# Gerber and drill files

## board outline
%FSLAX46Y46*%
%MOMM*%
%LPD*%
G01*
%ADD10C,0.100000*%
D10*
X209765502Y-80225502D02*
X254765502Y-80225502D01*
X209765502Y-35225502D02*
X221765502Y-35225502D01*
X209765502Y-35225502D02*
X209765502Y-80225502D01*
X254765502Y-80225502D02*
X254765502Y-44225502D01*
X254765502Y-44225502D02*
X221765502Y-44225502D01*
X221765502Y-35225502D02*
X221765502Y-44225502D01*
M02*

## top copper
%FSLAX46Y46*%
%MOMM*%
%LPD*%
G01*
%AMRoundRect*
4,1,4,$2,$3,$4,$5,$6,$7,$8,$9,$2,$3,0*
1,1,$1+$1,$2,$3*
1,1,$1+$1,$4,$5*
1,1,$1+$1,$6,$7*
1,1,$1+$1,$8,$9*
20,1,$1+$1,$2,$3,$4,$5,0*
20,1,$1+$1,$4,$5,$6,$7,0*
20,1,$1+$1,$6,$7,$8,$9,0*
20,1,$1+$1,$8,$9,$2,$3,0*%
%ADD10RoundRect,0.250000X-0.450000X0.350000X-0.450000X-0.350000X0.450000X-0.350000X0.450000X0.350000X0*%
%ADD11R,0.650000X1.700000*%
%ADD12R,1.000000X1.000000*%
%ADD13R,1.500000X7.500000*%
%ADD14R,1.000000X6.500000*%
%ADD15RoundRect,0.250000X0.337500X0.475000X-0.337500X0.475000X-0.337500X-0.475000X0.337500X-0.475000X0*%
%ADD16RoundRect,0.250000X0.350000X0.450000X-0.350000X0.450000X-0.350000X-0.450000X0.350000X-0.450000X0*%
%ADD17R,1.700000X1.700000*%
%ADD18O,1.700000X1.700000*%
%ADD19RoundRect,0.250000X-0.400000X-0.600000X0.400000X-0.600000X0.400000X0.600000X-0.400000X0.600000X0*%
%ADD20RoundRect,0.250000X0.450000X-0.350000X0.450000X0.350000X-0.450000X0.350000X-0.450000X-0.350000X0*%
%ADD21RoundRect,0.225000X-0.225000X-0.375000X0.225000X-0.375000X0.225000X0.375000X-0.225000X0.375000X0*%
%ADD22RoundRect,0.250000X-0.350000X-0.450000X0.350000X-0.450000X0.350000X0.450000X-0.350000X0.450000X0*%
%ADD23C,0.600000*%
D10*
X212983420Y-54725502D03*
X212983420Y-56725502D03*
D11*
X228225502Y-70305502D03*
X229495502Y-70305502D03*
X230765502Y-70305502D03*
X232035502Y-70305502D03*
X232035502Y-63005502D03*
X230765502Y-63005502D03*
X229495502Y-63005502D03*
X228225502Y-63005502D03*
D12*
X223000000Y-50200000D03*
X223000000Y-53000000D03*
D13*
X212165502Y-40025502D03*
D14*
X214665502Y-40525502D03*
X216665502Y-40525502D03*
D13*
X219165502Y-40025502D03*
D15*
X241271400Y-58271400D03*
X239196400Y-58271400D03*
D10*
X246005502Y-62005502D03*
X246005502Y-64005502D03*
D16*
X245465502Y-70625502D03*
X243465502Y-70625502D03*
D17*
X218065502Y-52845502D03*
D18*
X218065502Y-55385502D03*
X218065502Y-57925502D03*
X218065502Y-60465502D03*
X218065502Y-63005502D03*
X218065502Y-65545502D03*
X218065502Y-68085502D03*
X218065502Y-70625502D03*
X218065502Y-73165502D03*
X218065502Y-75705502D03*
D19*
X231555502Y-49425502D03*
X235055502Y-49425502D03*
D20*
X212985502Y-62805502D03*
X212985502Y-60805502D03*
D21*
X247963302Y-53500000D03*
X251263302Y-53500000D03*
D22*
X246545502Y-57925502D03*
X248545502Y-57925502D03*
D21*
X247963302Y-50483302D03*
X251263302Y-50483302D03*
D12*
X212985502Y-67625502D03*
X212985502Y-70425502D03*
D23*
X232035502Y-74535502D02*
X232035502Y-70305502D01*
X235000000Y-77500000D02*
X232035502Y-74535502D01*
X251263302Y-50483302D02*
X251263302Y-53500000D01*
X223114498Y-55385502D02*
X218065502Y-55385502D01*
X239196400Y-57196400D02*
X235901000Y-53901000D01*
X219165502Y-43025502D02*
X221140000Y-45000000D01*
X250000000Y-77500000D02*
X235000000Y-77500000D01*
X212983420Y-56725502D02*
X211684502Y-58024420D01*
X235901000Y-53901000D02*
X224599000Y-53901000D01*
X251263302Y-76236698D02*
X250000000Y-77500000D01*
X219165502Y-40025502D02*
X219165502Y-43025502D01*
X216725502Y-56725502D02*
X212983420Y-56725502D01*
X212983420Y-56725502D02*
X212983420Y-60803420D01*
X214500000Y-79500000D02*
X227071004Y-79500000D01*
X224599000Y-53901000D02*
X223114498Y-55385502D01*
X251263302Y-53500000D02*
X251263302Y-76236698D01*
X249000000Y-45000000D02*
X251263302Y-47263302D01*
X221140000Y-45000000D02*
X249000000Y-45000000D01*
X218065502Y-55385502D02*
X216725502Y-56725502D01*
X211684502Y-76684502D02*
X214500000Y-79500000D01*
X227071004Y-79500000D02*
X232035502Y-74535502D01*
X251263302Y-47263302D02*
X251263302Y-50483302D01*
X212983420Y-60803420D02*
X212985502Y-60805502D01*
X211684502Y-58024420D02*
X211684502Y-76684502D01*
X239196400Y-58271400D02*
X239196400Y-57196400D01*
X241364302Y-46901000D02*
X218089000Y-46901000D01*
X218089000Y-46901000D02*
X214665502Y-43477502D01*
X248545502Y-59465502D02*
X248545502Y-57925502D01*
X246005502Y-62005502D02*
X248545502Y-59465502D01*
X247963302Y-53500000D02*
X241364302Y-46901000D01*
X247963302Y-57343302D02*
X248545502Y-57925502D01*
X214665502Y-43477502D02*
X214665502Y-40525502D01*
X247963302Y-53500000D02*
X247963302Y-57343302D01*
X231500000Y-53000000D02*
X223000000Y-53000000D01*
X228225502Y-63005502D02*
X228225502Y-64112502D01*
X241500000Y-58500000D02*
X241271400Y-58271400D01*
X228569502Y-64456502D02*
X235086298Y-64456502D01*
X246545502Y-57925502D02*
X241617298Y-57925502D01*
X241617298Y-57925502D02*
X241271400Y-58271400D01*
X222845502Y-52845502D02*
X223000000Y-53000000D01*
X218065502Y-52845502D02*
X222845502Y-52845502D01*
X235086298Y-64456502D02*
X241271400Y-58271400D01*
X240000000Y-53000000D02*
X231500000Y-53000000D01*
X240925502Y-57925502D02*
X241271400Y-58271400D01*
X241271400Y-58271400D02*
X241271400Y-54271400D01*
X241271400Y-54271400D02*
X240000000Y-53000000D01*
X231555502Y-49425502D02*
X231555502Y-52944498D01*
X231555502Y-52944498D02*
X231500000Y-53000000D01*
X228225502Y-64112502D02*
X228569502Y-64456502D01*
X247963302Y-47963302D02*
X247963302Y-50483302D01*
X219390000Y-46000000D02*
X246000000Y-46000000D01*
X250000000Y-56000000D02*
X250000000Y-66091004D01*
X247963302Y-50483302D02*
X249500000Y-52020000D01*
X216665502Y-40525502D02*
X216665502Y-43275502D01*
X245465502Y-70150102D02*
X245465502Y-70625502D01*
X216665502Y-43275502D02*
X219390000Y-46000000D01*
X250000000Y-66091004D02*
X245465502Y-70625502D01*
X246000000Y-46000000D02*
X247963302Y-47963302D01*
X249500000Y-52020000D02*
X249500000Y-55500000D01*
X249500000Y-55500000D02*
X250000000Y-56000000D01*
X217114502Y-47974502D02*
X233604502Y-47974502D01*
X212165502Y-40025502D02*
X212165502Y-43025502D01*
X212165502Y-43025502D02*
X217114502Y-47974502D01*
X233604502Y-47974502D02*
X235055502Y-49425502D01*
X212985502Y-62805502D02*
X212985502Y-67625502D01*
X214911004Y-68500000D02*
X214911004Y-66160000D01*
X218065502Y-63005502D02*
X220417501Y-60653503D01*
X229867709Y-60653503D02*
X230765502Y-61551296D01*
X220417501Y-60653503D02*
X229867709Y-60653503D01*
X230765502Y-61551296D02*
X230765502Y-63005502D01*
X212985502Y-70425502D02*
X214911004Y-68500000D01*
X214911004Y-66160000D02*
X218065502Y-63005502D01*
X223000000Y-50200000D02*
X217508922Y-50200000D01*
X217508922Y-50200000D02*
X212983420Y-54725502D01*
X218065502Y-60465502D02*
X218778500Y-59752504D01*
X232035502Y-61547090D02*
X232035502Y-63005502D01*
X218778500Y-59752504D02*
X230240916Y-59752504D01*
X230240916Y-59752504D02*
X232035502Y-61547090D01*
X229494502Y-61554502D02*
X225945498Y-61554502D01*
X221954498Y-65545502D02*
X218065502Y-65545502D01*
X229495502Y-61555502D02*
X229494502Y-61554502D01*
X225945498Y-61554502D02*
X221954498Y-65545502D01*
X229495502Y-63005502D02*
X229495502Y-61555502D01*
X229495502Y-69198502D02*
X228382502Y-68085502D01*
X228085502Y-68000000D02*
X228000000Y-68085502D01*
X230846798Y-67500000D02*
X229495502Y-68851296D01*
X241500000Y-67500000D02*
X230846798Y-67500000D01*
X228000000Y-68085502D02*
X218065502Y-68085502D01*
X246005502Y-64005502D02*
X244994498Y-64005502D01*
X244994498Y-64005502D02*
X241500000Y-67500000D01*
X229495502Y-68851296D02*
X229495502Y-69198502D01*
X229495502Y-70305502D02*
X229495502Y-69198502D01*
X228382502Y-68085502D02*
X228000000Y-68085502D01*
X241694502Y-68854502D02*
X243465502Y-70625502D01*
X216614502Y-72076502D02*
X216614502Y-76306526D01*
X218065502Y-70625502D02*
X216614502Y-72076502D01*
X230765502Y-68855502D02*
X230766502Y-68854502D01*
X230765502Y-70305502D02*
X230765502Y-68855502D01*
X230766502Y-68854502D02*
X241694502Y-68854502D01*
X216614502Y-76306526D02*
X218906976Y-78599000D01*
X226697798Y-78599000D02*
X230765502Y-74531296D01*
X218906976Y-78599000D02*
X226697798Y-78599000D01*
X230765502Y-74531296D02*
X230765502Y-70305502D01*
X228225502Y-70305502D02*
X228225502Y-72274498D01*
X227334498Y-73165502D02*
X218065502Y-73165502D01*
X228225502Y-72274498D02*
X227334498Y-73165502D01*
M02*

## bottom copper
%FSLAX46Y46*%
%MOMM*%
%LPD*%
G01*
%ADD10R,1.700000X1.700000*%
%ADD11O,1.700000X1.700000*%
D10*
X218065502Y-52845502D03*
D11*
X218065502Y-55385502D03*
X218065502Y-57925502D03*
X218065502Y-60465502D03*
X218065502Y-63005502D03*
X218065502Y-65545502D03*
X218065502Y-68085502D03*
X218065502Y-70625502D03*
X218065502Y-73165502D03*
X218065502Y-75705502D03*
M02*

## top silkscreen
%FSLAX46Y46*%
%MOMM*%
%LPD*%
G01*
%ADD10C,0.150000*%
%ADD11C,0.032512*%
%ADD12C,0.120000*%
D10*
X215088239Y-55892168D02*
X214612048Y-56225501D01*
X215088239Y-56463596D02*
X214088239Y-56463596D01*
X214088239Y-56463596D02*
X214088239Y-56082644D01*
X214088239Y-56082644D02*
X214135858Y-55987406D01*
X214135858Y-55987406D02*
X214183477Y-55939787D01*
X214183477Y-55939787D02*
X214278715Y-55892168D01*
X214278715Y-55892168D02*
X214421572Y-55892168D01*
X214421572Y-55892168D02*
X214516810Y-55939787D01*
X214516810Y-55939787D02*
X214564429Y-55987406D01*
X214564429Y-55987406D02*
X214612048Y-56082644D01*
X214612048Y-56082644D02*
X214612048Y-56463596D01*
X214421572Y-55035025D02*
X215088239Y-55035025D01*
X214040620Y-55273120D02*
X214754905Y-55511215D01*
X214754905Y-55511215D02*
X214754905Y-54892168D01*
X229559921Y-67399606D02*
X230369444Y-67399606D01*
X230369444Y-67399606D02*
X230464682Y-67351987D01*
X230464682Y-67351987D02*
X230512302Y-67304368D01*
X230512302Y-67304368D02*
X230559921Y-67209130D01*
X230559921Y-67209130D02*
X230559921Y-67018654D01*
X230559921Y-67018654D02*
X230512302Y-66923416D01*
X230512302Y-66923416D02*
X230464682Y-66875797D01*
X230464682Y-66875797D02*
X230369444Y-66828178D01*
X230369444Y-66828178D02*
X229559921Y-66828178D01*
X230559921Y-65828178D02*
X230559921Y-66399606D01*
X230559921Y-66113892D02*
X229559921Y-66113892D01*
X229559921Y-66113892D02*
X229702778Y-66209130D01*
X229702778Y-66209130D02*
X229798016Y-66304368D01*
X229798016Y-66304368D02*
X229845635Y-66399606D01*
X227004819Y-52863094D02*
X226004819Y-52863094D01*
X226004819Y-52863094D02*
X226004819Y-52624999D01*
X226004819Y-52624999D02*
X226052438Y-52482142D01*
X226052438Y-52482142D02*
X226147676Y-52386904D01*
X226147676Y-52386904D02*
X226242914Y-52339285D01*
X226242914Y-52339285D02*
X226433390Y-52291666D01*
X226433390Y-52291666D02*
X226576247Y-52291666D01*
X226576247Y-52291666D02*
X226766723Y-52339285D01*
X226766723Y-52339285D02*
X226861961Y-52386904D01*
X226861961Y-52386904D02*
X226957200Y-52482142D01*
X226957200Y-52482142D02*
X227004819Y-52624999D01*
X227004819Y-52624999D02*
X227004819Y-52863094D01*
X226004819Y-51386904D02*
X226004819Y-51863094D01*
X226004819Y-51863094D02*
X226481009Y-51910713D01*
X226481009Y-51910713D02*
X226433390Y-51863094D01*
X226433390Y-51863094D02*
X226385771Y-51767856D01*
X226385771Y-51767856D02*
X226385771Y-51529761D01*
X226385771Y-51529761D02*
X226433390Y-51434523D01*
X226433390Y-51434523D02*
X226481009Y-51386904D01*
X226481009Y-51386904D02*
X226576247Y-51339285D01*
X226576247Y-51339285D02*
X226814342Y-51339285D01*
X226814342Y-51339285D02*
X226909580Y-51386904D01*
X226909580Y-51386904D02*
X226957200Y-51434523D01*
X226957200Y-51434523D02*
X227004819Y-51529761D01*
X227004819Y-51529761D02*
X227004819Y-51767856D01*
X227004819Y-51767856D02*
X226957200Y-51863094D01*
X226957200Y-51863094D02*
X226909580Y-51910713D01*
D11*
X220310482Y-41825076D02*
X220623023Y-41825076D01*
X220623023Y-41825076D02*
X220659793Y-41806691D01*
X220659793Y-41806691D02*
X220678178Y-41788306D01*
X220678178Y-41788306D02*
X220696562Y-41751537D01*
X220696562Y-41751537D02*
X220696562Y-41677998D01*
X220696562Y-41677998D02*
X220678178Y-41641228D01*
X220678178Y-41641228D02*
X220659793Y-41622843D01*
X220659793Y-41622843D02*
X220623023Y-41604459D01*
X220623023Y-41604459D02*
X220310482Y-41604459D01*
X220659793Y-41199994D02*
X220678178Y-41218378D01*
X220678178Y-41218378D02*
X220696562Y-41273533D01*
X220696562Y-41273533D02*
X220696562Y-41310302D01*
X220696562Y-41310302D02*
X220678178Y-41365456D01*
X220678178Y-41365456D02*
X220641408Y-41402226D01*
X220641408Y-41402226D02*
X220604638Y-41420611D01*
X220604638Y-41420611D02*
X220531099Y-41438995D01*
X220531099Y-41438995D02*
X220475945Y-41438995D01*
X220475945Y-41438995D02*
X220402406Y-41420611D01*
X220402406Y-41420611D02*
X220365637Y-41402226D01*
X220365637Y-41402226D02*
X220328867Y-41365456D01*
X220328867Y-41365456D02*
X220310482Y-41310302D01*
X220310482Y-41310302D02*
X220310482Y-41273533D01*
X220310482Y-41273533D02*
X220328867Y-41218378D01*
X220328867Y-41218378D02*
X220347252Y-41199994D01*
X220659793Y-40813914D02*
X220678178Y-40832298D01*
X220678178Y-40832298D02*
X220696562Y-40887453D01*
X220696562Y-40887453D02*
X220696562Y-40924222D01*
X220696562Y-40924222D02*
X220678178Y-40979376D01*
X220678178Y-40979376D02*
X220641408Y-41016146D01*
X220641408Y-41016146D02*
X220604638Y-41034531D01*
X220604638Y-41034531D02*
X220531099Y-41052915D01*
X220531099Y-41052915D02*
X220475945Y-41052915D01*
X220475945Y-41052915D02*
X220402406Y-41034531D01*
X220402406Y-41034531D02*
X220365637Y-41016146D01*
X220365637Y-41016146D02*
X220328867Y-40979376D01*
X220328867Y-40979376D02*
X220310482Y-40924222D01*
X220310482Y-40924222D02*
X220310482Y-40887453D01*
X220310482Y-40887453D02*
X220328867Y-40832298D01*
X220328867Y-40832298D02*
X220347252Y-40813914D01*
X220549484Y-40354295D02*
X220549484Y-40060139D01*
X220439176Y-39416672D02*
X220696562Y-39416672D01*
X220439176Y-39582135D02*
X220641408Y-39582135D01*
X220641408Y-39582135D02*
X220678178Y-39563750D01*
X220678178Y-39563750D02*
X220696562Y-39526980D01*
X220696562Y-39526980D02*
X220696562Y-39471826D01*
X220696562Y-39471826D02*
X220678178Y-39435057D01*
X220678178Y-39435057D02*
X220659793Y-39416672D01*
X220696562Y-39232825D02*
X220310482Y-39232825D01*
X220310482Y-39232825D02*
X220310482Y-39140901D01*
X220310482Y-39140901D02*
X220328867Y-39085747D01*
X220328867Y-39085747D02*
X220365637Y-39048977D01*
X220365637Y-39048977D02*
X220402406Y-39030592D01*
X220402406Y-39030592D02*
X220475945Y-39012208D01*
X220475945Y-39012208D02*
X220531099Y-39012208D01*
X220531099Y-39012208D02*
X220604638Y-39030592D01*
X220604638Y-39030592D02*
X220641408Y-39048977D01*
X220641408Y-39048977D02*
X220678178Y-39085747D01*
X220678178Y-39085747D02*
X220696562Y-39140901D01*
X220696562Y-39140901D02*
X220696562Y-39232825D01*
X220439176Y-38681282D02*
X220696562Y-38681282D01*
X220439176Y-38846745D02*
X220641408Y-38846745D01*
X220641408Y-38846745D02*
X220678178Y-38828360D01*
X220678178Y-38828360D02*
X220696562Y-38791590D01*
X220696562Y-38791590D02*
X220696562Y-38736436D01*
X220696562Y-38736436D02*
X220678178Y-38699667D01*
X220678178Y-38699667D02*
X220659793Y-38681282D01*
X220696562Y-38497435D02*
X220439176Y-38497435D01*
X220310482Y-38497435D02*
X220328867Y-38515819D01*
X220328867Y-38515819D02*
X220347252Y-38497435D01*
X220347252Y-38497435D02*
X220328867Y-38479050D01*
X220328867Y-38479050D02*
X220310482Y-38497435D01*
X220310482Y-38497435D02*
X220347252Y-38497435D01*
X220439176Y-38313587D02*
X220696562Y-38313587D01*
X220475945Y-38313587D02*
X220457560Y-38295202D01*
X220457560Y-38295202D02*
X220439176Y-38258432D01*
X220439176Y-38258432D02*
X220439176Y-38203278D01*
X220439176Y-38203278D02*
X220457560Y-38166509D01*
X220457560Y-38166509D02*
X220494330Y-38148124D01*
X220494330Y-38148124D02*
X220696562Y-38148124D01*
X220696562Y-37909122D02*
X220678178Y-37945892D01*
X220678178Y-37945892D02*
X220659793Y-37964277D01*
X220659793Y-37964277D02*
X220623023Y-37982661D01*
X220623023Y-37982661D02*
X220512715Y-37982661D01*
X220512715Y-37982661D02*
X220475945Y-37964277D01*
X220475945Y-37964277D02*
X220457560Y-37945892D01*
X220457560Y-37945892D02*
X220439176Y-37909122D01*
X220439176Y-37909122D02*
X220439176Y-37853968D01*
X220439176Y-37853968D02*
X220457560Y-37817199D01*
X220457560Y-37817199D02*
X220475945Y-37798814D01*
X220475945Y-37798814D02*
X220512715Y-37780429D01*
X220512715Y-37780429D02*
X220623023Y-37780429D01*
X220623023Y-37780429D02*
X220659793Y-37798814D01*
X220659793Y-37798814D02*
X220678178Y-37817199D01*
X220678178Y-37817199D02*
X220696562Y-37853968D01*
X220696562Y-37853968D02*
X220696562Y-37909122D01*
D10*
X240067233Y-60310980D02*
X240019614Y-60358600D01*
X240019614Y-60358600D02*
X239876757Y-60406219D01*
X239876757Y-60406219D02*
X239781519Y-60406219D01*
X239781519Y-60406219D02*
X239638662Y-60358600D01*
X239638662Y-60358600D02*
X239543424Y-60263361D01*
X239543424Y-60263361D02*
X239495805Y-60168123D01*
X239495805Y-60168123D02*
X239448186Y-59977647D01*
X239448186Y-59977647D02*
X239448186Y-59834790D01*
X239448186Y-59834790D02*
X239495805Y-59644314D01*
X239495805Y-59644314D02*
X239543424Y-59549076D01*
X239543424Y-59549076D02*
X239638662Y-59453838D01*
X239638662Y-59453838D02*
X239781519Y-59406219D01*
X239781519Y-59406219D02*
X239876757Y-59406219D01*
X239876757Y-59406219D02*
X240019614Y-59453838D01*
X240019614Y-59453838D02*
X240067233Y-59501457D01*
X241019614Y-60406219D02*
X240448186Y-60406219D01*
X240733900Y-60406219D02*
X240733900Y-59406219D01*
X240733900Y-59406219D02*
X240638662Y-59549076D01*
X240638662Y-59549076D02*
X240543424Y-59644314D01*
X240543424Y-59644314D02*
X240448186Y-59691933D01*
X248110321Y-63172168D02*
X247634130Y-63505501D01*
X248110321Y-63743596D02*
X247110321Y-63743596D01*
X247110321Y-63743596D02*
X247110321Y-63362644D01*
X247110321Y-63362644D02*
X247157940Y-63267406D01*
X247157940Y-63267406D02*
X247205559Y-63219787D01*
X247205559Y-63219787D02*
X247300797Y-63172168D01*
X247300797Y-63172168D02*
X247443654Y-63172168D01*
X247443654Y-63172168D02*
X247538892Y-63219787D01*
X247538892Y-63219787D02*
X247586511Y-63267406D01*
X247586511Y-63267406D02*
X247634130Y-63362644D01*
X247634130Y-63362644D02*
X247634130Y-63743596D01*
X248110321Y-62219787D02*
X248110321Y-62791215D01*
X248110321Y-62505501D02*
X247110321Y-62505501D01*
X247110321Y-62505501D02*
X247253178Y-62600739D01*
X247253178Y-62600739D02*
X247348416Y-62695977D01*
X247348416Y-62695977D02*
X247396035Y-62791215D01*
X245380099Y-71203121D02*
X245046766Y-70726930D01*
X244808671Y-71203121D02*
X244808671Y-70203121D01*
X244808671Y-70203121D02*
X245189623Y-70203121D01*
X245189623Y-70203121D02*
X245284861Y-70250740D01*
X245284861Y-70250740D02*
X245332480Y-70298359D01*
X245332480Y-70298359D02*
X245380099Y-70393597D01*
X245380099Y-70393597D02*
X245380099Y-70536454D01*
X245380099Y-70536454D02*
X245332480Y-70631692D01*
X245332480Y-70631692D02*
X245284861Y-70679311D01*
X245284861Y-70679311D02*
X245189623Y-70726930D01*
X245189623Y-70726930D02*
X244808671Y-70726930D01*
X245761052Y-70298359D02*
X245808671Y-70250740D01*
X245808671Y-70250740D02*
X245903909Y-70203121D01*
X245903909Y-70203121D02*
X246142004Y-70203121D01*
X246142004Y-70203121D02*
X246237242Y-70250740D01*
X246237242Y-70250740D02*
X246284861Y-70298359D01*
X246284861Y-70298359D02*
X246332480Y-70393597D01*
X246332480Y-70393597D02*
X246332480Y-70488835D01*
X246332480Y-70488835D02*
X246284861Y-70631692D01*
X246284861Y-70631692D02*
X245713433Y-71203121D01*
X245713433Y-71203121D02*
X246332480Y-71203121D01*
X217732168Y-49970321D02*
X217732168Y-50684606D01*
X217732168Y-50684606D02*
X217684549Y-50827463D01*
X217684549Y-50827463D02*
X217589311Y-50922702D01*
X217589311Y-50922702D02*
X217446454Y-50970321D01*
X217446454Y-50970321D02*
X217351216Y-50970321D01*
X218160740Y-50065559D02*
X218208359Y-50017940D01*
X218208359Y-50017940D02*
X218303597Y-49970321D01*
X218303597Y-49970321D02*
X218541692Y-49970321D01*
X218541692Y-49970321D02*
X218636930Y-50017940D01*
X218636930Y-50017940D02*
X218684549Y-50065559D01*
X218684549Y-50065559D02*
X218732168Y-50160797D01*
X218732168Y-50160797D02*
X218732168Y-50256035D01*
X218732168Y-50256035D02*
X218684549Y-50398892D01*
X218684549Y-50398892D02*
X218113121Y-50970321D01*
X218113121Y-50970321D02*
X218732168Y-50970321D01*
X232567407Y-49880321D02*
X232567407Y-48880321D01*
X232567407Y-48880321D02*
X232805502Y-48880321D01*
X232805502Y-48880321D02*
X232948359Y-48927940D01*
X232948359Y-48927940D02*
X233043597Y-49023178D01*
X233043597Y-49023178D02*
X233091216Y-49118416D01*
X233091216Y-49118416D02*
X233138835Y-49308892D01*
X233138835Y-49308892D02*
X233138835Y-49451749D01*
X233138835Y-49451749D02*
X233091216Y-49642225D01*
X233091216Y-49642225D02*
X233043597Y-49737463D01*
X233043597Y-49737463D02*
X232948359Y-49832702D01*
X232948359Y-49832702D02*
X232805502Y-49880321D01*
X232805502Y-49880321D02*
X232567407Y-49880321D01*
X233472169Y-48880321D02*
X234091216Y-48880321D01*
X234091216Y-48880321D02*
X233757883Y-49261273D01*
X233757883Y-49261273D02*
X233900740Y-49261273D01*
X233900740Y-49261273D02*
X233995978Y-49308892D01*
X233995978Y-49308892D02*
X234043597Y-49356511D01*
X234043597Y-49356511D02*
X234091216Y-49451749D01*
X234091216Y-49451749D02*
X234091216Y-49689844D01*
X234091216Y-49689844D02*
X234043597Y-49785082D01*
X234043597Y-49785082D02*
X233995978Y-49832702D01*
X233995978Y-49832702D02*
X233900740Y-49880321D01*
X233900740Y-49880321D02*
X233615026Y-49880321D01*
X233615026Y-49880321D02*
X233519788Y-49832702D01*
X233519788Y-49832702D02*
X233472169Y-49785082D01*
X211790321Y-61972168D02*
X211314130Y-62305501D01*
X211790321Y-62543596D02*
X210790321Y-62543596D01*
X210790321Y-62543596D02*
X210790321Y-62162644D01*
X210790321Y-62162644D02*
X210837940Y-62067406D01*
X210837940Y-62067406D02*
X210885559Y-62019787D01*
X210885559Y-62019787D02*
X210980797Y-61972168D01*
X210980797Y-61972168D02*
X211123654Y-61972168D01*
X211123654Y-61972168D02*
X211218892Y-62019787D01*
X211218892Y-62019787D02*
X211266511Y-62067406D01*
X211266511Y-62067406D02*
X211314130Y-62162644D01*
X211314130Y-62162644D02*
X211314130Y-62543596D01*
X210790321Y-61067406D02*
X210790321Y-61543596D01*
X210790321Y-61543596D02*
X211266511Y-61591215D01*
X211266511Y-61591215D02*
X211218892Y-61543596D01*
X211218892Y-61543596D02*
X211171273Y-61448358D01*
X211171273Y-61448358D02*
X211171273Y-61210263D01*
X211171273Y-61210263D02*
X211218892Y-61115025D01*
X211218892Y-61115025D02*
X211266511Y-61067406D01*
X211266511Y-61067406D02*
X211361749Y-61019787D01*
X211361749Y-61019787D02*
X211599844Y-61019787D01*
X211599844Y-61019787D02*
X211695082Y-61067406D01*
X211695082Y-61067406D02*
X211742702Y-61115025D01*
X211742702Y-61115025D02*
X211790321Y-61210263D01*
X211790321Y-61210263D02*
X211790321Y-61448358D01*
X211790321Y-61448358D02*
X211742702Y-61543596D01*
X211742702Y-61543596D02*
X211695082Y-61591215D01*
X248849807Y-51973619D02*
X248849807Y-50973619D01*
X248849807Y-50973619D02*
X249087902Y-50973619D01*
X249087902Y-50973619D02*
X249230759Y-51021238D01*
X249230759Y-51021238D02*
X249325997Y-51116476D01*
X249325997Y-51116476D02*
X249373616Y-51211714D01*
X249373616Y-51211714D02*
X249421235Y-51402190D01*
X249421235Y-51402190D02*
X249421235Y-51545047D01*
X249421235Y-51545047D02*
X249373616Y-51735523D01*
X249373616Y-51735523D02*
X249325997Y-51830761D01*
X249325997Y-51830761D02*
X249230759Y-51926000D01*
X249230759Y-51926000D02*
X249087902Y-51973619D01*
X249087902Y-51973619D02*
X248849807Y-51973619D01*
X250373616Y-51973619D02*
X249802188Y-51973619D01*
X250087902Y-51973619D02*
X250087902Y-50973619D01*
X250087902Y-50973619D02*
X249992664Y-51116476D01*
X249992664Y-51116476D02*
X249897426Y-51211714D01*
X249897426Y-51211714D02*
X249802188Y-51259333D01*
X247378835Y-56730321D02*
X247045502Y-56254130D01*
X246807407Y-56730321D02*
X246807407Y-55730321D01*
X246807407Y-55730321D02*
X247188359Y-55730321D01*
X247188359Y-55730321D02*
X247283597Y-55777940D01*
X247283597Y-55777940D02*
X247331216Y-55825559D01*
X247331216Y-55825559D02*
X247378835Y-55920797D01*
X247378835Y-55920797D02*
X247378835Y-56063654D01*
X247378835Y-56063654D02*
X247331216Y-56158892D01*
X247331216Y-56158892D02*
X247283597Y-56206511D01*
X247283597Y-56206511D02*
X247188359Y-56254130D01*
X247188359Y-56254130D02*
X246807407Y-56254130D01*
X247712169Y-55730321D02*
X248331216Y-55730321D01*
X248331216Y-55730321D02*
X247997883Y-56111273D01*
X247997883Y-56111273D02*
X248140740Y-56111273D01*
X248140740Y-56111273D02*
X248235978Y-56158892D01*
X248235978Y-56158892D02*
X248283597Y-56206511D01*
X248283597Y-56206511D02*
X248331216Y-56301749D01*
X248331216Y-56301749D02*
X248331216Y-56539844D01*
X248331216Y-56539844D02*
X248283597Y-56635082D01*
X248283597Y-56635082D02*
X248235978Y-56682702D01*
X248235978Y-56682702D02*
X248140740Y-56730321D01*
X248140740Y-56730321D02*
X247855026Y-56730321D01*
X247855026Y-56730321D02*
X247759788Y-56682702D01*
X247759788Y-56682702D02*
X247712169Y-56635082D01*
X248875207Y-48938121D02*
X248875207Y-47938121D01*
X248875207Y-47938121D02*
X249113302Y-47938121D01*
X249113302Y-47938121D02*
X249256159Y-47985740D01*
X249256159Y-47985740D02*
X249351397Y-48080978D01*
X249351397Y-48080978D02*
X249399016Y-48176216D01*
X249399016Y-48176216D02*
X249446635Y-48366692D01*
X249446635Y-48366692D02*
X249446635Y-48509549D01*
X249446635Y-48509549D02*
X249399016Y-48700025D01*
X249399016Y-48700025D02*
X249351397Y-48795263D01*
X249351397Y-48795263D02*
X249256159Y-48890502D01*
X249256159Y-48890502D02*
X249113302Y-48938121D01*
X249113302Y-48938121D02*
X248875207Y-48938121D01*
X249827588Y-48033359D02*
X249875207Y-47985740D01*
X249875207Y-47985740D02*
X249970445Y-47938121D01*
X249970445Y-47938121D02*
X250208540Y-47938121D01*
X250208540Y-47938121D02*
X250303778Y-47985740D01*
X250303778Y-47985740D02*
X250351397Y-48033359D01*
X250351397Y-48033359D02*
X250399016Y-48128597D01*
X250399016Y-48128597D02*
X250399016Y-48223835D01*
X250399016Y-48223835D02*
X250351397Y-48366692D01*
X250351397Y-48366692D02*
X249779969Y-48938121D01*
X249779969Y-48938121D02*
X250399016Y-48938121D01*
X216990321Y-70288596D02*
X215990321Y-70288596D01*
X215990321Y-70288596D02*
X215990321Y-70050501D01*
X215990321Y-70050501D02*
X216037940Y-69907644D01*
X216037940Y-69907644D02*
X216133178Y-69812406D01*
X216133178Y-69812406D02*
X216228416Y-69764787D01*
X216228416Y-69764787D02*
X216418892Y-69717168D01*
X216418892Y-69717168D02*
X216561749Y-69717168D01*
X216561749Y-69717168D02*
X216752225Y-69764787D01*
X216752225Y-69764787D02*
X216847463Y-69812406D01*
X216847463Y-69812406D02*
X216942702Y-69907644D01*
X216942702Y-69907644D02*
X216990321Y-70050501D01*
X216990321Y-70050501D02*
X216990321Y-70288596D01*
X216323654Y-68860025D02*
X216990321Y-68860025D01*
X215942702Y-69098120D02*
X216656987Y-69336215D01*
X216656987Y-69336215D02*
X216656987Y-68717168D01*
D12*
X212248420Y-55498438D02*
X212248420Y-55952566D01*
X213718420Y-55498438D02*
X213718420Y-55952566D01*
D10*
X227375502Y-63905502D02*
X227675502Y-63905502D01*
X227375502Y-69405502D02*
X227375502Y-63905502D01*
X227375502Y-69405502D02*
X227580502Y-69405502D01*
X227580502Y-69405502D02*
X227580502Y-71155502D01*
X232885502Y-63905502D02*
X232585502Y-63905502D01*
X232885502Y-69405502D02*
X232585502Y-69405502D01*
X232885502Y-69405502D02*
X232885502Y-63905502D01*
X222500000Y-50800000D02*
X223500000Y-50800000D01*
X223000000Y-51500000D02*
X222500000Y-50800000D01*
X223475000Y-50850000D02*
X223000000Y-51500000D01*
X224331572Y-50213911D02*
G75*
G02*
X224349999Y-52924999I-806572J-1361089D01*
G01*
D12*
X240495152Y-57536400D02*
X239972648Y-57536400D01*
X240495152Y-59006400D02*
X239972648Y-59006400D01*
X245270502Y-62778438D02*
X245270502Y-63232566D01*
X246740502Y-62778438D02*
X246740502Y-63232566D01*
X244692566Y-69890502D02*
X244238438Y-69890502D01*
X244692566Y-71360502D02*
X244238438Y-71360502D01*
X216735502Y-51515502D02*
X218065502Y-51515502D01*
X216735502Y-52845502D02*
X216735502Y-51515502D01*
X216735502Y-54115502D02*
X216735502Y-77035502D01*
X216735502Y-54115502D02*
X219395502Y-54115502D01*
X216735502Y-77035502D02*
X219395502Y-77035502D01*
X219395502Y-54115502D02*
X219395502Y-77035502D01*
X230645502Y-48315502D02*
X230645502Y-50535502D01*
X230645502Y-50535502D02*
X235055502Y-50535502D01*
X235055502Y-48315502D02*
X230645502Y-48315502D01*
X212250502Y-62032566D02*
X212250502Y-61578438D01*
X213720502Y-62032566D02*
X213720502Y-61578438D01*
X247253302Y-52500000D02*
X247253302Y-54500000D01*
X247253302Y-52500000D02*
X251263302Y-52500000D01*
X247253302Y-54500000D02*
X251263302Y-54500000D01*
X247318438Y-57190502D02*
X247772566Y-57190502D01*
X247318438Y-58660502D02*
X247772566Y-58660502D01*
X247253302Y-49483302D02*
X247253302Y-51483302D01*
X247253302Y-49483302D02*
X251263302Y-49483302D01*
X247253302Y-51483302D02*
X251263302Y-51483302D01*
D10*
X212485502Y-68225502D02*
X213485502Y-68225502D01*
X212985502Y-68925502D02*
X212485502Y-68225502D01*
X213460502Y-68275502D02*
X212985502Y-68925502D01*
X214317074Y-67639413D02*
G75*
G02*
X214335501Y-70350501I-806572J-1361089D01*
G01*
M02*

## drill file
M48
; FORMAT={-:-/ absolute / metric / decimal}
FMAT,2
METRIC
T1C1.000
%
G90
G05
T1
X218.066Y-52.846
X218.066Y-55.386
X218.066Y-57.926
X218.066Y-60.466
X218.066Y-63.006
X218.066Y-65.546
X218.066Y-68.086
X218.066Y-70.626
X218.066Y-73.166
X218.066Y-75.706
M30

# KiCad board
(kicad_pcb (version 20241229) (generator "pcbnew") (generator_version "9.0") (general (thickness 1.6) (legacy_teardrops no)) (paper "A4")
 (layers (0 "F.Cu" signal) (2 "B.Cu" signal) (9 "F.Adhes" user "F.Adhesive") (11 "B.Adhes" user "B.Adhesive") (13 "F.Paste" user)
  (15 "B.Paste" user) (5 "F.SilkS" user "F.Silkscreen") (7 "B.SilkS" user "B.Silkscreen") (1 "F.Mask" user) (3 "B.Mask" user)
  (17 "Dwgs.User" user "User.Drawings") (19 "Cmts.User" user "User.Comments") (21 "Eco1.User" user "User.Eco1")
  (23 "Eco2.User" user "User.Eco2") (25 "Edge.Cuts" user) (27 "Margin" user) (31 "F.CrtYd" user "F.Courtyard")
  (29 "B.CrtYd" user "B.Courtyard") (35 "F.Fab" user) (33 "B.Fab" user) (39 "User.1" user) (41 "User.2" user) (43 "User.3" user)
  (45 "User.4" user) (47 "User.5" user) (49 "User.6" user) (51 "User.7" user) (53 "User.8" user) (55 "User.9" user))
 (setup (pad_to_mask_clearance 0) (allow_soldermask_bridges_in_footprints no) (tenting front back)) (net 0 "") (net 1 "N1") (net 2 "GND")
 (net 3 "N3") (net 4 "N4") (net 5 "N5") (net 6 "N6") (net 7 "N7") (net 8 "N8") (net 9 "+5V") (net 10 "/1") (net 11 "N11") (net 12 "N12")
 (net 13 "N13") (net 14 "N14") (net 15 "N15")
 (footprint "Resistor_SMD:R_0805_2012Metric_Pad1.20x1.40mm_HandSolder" (layer "F.Cu") (at 212.98342 55.725502 -90)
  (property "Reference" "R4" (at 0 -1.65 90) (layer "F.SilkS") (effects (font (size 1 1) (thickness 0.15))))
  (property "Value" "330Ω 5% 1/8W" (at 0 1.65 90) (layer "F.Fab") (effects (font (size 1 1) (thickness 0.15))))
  (fp_line (start -0.227064 0.735) (end 0.227064 0.735) (stroke (width 0.12) (type solid)) (layer "F.SilkS"))
  (fp_line (start -0.227064 -0.735) (end 0.227064 -0.735) (stroke (width 0.12) (type solid)) (layer "F.SilkS"))
  (pad "1" smd roundrect (at -1 0 270) (size 1.2 1.4) (layers "F.Cu" "F.Mask" "F.Paste") (roundrect_rratio 0.208333) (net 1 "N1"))
  (pad "2" smd roundrect (at 1 0 270) (size 1.2 1.4) (layers "F.Cu" "F.Mask" "F.Paste") (roundrect_rratio 0.208333) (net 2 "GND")))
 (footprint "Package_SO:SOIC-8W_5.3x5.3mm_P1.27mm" (layer "F.Cu") (at 230.130502 66.655502 90)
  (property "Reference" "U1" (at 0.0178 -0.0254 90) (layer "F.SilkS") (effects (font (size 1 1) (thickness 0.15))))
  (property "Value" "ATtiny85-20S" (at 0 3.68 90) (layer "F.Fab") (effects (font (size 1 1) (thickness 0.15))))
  (fp_line (start 2.75 -2.755) (end 2.75 -2.455) (stroke (width 0.15) (type solid)) (layer "F.SilkS"))
  (fp_line (start -2.75 -2.755) (end 2.75 -2.755) (stroke (width 0.15) (type solid)) (layer "F.SilkS"))
  (fp_line (start -2.75 -2.755) (end -2.75 -2.55) (stroke (width 0.15) (type solid)) (layer "F.SilkS"))
  (fp_line (start -2.75 -2.55) (end -4.5 -2.55) (stroke (width 0.15) (type solid)) (layer "F.SilkS"))
  (fp_line (start 2.75 2.755) (end 2.75 2.455) (stroke (width 0.15) (type solid)) (layer "F.SilkS"))
  (fp_line (start -2.75 2.755) (end -2.75 2.455) (stroke (width 0.15) (type solid)) (layer "F.SilkS"))
  (fp_line (start -2.75 2.755) (end 2.75 2.755) (stroke (width 0.15) (type solid)) (layer "F.SilkS"))
  (pad "1" smd rect (at -3.65 -1.905 90) (size 1.7 0.65) (layers "F.Cu" "F.Mask" "F.Paste") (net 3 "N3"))
  (pad "2" smd rect (at -3.65 -0.635 90) (size 1.7 0.65) (layers "F.Cu" "F.Mask" "F.Paste") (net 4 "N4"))
  (pad "3" smd rect (at -3.65 0.635 90) (size 1.7 0.65) (layers "F.Cu" "F.Mask" "F.Paste") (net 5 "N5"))
  (pad "4" smd rect (at -3.65 1.905 90) (size 1.7 0.65) (layers "F.Cu" "F.Mask" "F.Paste") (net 2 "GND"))
  (pad "5" smd rect (at 3.65 1.905 90) (size 1.7 0.65) (layers "F.Cu" "F.Mask" "F.Paste") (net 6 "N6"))
  (pad "6" smd rect (at 3.65 0.635 90) (size 1.7 0.65) (layers "F.Cu" "F.Mask" "F.Paste") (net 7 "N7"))
  (pad "7" smd rect (at 3.65 -0.635 90) (size 1.7 0.65) (layers "F.Cu" "F.Mask" "F.Paste") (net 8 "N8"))
  (pad "8" smd rect (at 3.65 -1.905 90) (size 1.7 0.65) (layers "F.Cu" "F.Mask" "F.Paste") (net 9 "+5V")))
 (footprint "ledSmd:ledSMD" (layer "F.Cu") (at 223 52 -90)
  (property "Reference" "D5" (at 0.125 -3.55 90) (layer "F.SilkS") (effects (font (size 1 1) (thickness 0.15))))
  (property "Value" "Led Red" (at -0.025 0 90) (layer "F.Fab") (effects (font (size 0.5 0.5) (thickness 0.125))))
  (fp_line (start -1.2 0.5) (end -1.2 -0.5) (stroke (width 0.15) (type solid)) (layer "F.SilkS"))
  (fp_line (start -0.5 0) (end -1.2 0.5) (stroke (width 0.15) (type solid)) (layer "F.SilkS"))
  (fp_line (start -1.15 -0.475) (end -0.5 0) (stroke (width 0.15) (type solid)) (layer "F.SilkS"))
  (fp_arc (start -1.786089 -1.331572) (mid -0.435753 -2.107089) (end 0.924999 -1.349999) (stroke (width 0.15) (type solid))
   (layer "F.SilkS"))
  (pad "1" smd rect (at -1.8 0 270) (size 1 1) (layers "F.Cu" "F.Mask" "F.Paste") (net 1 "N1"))
  (pad "2" smd rect (at 1 0 270) (size 1 1) (layers "F.Cu" "F.Mask" "F.Paste") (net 9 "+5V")))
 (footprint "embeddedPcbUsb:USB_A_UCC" (layer "F.Cu") (at 215.665502 40.225502 -90)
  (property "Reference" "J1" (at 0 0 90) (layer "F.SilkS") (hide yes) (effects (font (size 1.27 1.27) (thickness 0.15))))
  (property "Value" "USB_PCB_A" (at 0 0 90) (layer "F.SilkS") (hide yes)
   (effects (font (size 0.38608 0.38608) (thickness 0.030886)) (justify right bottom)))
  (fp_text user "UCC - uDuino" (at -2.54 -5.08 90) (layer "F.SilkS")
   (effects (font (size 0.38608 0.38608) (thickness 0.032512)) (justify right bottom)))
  (pad "1" smd rect (at -0.2 3.5 270) (size 7.5 1.5) (layers "F.Cu" "F.Mask" "F.Paste") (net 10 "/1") (solder_mask_margin 0.1016))
  (pad "2" smd rect (at 0.3 1 270) (size 6.5 1) (layers "F.Cu" "F.Mask" "F.Paste") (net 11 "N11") (solder_mask_margin 0.1016))
  (pad "3" smd rect (at 0.3 -1 270) (size 6.5 1) (layers "F.Cu" "F.Mask" "F.Paste") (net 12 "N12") (solder_mask_margin 0.1016))
  (pad "4" smd rect (at -0.2 -3.5 270) (size 7.5 1.5) (layers "F.Cu" "F.Mask" "F.Paste") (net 2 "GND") (solder_mask_margin 0.1016)))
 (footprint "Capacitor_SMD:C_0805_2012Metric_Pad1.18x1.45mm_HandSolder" (layer "F.Cu") (at 240.2339 58.2714 180)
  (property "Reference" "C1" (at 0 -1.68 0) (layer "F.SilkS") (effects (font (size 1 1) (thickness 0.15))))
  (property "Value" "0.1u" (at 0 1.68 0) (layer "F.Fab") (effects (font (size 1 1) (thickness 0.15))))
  (fp_line (start -0.261252 0.735) (end 0.261252 0.735) (stroke (width 0.12) (type solid)) (layer "F.SilkS"))
  (fp_line (start -0.261252 -0.735) (end 0.261252 -0.735) (stroke (width 0.12) (type solid)) (layer "F.SilkS"))
  (pad "1" smd roundrect (at -1.0375 0 180) (size 1.175 1.45) (layers "F.Cu" "F.Mask" "F.Paste") (roundrect_rratio 0.212766) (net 9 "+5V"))
  (pad "2" smd roundrect (at 1.0375 0 180) (size 1.175 1.45) (layers "F.Cu" "F.Mask" "F.Paste") (roundrect_rratio 0.212766) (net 2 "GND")))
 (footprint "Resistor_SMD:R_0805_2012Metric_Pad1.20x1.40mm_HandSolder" (layer "F.Cu") (at 246.005502 63.005502 -90)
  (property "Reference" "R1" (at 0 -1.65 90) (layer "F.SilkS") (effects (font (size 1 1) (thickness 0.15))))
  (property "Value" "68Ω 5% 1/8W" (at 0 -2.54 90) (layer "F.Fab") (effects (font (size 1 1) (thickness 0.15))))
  (fp_line (start -0.227064 0.735) (end 0.227064 0.735) (stroke (width 0.12) (type solid)) (layer "F.SilkS"))
  (fp_line (start -0.227064 -0.735) (end 0.227064 -0.735) (stroke (width 0.12) (type solid)) (layer "F.SilkS"))
  (pad "1" smd roundrect (at -1 0 270) (size 1.2 1.4) (layers "F.Cu" "F.Mask" "F.Paste") (roundrect_rratio 0.208333) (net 11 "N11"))
  (pad "2" smd roundrect (at 1 0 270) (size 1.2 1.4) (layers "F.Cu" "F.Mask" "F.Paste") (roundrect_rratio 0.208333) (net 4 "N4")))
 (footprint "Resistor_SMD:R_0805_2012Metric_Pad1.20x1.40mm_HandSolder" (layer "F.Cu") (at 244.465502 70.625502 180)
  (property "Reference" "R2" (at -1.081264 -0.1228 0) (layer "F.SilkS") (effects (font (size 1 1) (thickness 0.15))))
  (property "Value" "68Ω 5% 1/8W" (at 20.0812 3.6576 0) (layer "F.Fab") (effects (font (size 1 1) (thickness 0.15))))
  (fp_line (start -0.227064 0.735) (end 0.227064 0.735) (stroke (width 0.12) (type solid)) (layer "F.SilkS"))
  (fp_line (start -0.227064 -0.735) (end 0.227064 -0.735) (stroke (width 0.12) (type solid)) (layer "F.SilkS"))
  (pad "1" smd roundrect (at -1 0 180) (size 1.2 1.4) (layers "F.Cu" "F.Mask" "F.Paste") (roundrect_rratio 0.208333) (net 12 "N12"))
  (pad "2" smd roundrect (at 1 0 180) (size 1.2 1.4) (layers "F.Cu" "F.Mask" "F.Paste") (roundrect_rratio 0.208333) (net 5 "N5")))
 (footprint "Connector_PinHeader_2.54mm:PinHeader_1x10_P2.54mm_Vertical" (layer "F.Cu") (at 218.065502 52.845502)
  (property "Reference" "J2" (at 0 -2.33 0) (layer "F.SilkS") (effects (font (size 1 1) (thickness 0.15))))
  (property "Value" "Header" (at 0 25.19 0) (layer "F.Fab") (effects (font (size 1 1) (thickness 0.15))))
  (fp_line (start -1.33 -1.33) (end 0 -1.33) (stroke (width 0.12) (type solid)) (layer "F.SilkS"))
  (fp_line (start -1.33 0) (end -1.33 -1.33) (stroke (width 0.12) (type solid)) (layer "F.SilkS"))
  (fp_line (start -1.33 1.27) (end -1.33 24.19) (stroke (width 0.12) (type solid)) (layer "F.SilkS"))
  (fp_line (start -1.33 1.27) (end 1.33 1.27) (stroke (width 0.12) (type solid)) (layer "F.SilkS"))
  (fp_line (start -1.33 24.19) (end 1.33 24.19) (stroke (width 0.12) (type solid)) (layer "F.SilkS"))
  (fp_line (start 1.33 1.27) (end 1.33 24.19) (stroke (width 0.12) (type solid)) (layer "F.SilkS"))
  (pad "1" thru_hole rect (at 0 0) (size 1.7 1.7) (drill 1) (layers "*.Cu" "*.Mask") (remove_unused_layers no) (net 9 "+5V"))
  (pad "2" thru_hole oval (at 0 2.54) (size 1.7 1.7) (drill 1) (layers "*.Cu" "*.Mask") (remove_unused_layers no) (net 2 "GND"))
  (pad "3" thru_hole oval (at 0 5.08) (size 1.7 1.7) (drill 1) (layers "*.Cu" "*.Mask") (remove_unused_layers no) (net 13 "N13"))
  (pad "4" thru_hole oval (at 0 7.62) (size 1.7 1.7) (drill 1) (layers "*.Cu" "*.Mask") (remove_unused_layers no) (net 6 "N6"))
  (pad "5" thru_hole oval (at 0 10.16) (size 1.7 1.7) (drill 1) (layers "*.Cu" "*.Mask") (remove_unused_layers no) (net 7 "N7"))
  (pad "6" thru_hole oval (at 0 12.7) (size 1.7 1.7) (drill 1) (layers "*.Cu" "*.Mask") (remove_unused_layers no) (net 8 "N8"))
  (pad "7" thru_hole oval (at 0 15.24) (size 1.7 1.7) (drill 1) (layers "*.Cu" "*.Mask") (remove_unused_layers no) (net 4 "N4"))
  (pad "8" thru_hole oval (at 0 17.78) (size 1.7 1.7) (drill 1) (layers "*.Cu" "*.Mask") (remove_unused_layers no) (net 5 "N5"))
  (pad "9" thru_hole oval (at 0 20.32) (size 1.7 1.7) (drill 1) (layers "*.Cu" "*.Mask") (remove_unused_layers no) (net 3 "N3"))
  (pad "10" thru_hole oval (at 0 22.86) (size 1.7 1.7) (drill 1) (layers "*.Cu" "*.Mask") (remove_unused_layers no) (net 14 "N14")))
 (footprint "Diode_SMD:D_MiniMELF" (layer "F.Cu") (at 233.305502 49.425502)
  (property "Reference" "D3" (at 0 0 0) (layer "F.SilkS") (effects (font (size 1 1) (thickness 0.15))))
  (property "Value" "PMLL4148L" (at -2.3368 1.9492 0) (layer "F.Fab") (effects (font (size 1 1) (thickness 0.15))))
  (fp_line (start -2.66 -1.11) (end -2.66 1.11) (stroke (width 0.12) (type solid)) (layer "F.SilkS"))
  (fp_line (start -2.66 1.11) (end 1.75 1.11) (stroke (width 0.12) (type solid)) (layer "F.SilkS"))
  (fp_line (start 1.75 -1.11) (end -2.66 -1.11) (stroke (width 0.12) (type solid)) (layer "F.SilkS"))
  (pad "1" smd roundrect (at -1.75 0) (size 1.3 1.7) (layers "F.Cu" "F.Mask" "F.Paste") (roundrect_rratio 0.1923076923) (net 9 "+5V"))
  (pad "2" smd roundrect (at 1.75 0) (size 1.3 1.7) (layers "F.Cu" "F.Mask" "F.Paste") (roundrect_rratio 0.1923076923) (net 10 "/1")))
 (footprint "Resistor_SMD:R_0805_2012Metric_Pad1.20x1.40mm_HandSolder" (layer "F.Cu") (at 212.985502 61.805502 90)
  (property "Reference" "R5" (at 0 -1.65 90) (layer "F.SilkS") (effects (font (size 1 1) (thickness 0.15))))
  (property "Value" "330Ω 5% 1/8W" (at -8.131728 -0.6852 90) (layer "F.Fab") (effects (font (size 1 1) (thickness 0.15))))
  (fp_line (start -0.227064 -0.735) (end 0.227064 -0.735) (stroke (width 0.12) (type solid)) (layer "F.SilkS"))
  (fp_line (start -0.227064 0.735) (end 0.227064 0.735) (stroke (width 0.12) (type solid)) (layer "F.SilkS"))
  (pad "1" smd roundrect (at -1 0 90) (size 1.2 1.4) (layers "F.Cu" "F.Mask" "F.Paste") (roundrect_rratio 0.208333) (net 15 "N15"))
  (pad "2" smd roundrect (at 1 0 90) (size 1.2 1.4) (layers "F.Cu" "F.Mask" "F.Paste") (roundrect_rratio 0.208333) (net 2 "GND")))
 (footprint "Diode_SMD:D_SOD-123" (layer "F.Cu") (at 249.613302 53.5)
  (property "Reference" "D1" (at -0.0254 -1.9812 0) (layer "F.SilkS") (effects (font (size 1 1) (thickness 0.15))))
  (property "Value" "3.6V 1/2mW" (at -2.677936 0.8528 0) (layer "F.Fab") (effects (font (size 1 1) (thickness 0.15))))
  (fp_line (start -2.36 -1) (end -2.36 1) (stroke (width 0.12) (type solid)) (layer "F.SilkS"))
  (fp_line (start -2.36 -1) (end 1.65 -1) (stroke (width 0.12) (type solid)) (layer "F.SilkS"))
  (fp_line (start -2.36 1) (end 1.65 1) (stroke (width 0.12) (type solid)) (layer "F.SilkS"))
  (pad "1" smd roundrect (at -1.65 0) (size 0.9 1.2) (layers "F.Cu" "F.Mask" "F.Paste") (roundrect_rratio 0.25) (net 11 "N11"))
  (pad "2" smd roundrect (at 1.65 0) (size 0.9 1.2) (layers "F.Cu" "F.Mask" "F.Paste") (roundrect_rratio 0.25) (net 2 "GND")))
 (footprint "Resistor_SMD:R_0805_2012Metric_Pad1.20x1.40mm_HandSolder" (layer "F.Cu") (at 247.545502 57.925502)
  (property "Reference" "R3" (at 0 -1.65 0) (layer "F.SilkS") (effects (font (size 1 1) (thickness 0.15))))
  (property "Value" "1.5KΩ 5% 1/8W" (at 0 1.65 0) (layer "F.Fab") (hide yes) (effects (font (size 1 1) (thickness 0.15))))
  (fp_line (start -0.227064 -0.735) (end 0.227064 -0.735) (stroke (width 0.12) (type solid)) (layer "F.SilkS"))
  (fp_line (start -0.227064 0.735) (end 0.227064 0.735) (stroke (width 0.12) (type solid)) (layer "F.SilkS"))
  (pad "1" smd roundrect (at -1 0) (size 1.2 1.4) (layers "F.Cu" "F.Mask" "F.Paste") (roundrect_rratio 0.208333) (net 9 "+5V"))
  (pad "2" smd roundrect (at 1 0) (size 1.2 1.4) (layers "F.Cu" "F.Mask" "F.Paste") (roundrect_rratio 0.208333) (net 11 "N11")))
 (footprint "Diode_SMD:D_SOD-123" (layer "F.Cu") (at 249.613302 50.483302)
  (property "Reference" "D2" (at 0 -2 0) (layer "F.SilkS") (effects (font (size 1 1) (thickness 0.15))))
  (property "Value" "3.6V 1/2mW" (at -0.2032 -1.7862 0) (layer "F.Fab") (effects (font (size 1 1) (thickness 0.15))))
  (fp_line (start -2.36 -1) (end -2.36 1) (stroke (width 0.12) (type solid)) (layer "F.SilkS"))
  (fp_line (start -2.36 -1) (end 1.65 -1) (stroke (width 0.12) (type solid)) (layer "F.SilkS"))
  (fp_line (start -2.36 1) (end 1.65 1) (stroke (width 0.12) (type solid)) (layer "F.SilkS"))
  (pad "1" smd roundrect (at -1.65 0) (size 0.9 1.2) (layers "F.Cu" "F.Mask" "F.Paste") (roundrect_rratio 0.25) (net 12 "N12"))
  (pad "2" smd roundrect (at 1.65 0) (size 0.9 1.2) (layers "F.Cu" "F.Mask" "F.Paste") (roundrect_rratio 0.25) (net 2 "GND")))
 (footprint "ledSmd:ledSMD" (layer "F.Cu") (at 212.985502 69.425502 -90)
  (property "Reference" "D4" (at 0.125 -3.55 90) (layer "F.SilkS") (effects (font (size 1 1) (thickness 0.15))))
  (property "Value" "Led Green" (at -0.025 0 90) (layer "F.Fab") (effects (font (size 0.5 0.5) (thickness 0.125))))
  (fp_line (start -1.2 0.5) (end -1.2 -0.5) (stroke (width 0.15) (type solid)) (layer "F.SilkS"))
  (fp_line (start -0.5 0) (end -1.2 0.5) (stroke (width 0.15) (type solid)) (layer "F.SilkS"))
  (fp_line (start -1.15 -0.475) (end -0.5 0) (stroke (width 0.15) (type solid)) (layer "F.SilkS"))
  (fp_arc (start -1.786089 -1.331572) (mid -0.435753 -2.107089) (end 0.924999 -1.349999) (stroke (width 0.15) (type solid))
   (layer "F.SilkS"))
  (pad "1" smd rect (at -1.8 0 270) (size 1 1) (layers "F.Cu" "F.Mask" "F.Paste") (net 15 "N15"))
  (pad "2" smd rect (at 1 0 270) (size 1 1) (layers "F.Cu" "F.Mask" "F.Paste") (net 7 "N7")))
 (gr_line (start 209.765502 80.225502) (end 254.765502 80.225502) (stroke (width 0.1) (type default)) (layer "Edge.Cuts"))
 (gr_line (start 209.765502 35.225502) (end 221.765502 35.225502) (stroke (width 0.1) (type default)) (layer "Edge.Cuts"))
 (gr_line (start 209.765502 35.225502) (end 209.765502 80.225502) (stroke (width 0.1) (type default)) (layer "Edge.Cuts"))
 (gr_line (start 254.765502 80.225502) (end 254.765502 44.225502) (stroke (width 0.1) (type default)) (layer "Edge.Cuts"))
 (gr_line (start 254.765502 44.225502) (end 221.765502 44.225502) (stroke (width 0.1) (type default)) (layer "Edge.Cuts"))
 (gr_line (start 221.765502 35.225502) (end 221.765502 44.225502) (stroke (width 0.1) (type default)) (layer "Edge.Cuts"))
 (segment (start 232.035502 74.535502) (end 232.035502 70.305502) (width 0.6) (layer "F.Cu") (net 2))
 (segment (start 235 77.5) (end 232.035502 74.535502) (width 0.6) (layer "F.Cu") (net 2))
 (segment (start 251.263302 50.483302) (end 251.263302 53.5) (width 0.6) (layer "F.Cu") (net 2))
 (segment (start 223.114498 55.385502) (end 218.065502 55.385502) (width 0.6) (layer "F.Cu") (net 2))
 (segment (start 239.1964 57.1964) (end 235.901 53.901) (width 0.6) (layer "F.Cu") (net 2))
 (segment (start 219.165502 43.025502) (end 221.14 45) (width 0.6) (layer "F.Cu") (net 2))
 (segment (start 250 77.5) (end 235 77.5) (width 0.6) (layer "F.Cu") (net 2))
 (segment (start 212.98342 56.725502) (end 211.684502 58.02442) (width 0.6) (layer "F.Cu") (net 2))
 (segment (start 235.901 53.901) (end 224.599 53.901) (width 0.6) (layer "F.Cu") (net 2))
 (segment (start 251.263302 76.236698) (end 250 77.5) (width 0.6) (layer "F.Cu") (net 2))
 (segment (start 219.165502 40.025502) (end 219.165502 43.025502) (width 0.6) (layer "F.Cu") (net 2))
 (segment (start 216.725502 56.725502) (end 212.98342 56.725502) (width 0.6) (layer "F.Cu") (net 2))
 (segment (start 212.98342 56.725502) (end 212.98342 60.80342) (width 0.6) (layer "F.Cu") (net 2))
 (segment (start 214.5 79.5) (end 227.071004 79.5) (width 0.6) (layer "F.Cu") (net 2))
 (segment (start 224.599 53.901) (end 223.114498 55.385502) (width 0.6) (layer "F.Cu") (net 2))
 (segment (start 251.263302 53.5) (end 251.263302 76.236698) (width 0.6) (layer "F.Cu") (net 2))
 (segment (start 249 45) (end 251.263302 47.263302) (width 0.6) (layer "F.Cu") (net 2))
 (segment (start 221.14 45) (end 249 45) (width 0.6) (layer "F.Cu") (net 2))
 (segment (start 218.065502 55.385502) (end 216.725502 56.725502) (width 0.6) (layer "F.Cu") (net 2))
 (segment (start 211.684502 76.684502) (end 214.5 79.5) (width 0.6) (layer "F.Cu") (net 2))
 (segment (start 227.071004 79.5) (end 232.035502 74.535502) (width 0.6) (layer "F.Cu") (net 2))
 (segment (start 251.263302 47.263302) (end 251.263302 50.483302) (width 0.6) (layer "F.Cu") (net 2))
 (segment (start 212.98342 60.80342) (end 212.985502 60.805502) (width 0.6) (layer "F.Cu") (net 2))
 (segment (start 211.684502 58.02442) (end 211.684502 76.684502) (width 0.6) (layer "F.Cu") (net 2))
 (segment (start 239.1964 58.2714) (end 239.1964 57.1964) (width 0.6) (layer "F.Cu") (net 2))
 (segment (start 241.364302 46.901) (end 218.089 46.901) (width 0.6) (layer "F.Cu") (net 11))
 (segment (start 218.089 46.901) (end 214.665502 43.477502) (width 0.6) (layer "F.Cu") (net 11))
 (segment (start 248.545502 59.465502) (end 248.545502 57.925502) (width 0.6) (layer "F.Cu") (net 11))
 (segment (start 246.005502 62.005502) (end 248.545502 59.465502) (width 0.6) (layer "F.Cu") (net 11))
 (segment (start 247.963302 53.5) (end 241.364302 46.901) (width 0.6) (layer "F.Cu") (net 11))
 (segment (start 247.963302 57.343302) (end 248.545502 57.925502) (width 0.6) (layer "F.Cu") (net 11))
 (segment (start 214.665502 43.477502) (end 214.665502 40.525502) (width 0.6) (layer "F.Cu") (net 11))
 (segment (start 247.963302 53.5) (end 247.963302 57.343302) (width 0.6) (layer "F.Cu") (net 11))
 (segment (start 231.5 53) (end 223 53) (width 0.6) (layer "F.Cu") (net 9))
 (segment (start 228.225502 63.005502) (end 228.225502 64.112502) (width 0.6) (layer "F.Cu") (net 9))
 (segment (start 241.5 58.5) (end 241.2714 58.2714) (width 0.6) (layer "F.Cu") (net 9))
 (segment (start 228.569502 64.456502) (end 235.086298 64.456502) (width 0.6) (layer "F.Cu") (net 9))
 (segment (start 246.545502 57.925502) (end 241.617298 57.925502) (width 0.6) (layer "F.Cu") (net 9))
 (segment (start 241.617298 57.925502) (end 241.2714 58.2714) (width 0.6) (layer "F.Cu") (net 9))
 (segment (start 222.845502 52.845502) (end 223 53) (width 0.6) (layer "F.Cu") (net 9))
 (segment (start 218.065502 52.845502) (end 222.845502 52.845502) (width 0.6) (layer "F.Cu") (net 9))
 (segment (start 235.086298 64.456502) (end 241.2714 58.2714) (width 0.6) (layer "F.Cu") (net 9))
 (segment (start 240 53) (end 231.5 53) (width 0.6) (layer "F.Cu") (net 9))
 (segment (start 240.925502 57.925502) (end 241.2714 58.2714) (width 0.6) (layer "F.Cu") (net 9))
 (segment (start 241.2714 58.2714) (end 241.2714 54.2714) (width 0.6) (layer "F.Cu") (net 9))
 (segment (start 241.2714 54.2714) (end 240 53) (width 0.6) (layer "F.Cu") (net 9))
 (segment (start 231.555502 49.425502) (end 231.555502 52.944498) (width 0.6) (layer "F.Cu") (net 9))
 (segment (start 231.555502 52.944498) (end 231.5 53) (width 0.6) (layer "F.Cu") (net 9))
 (segment (start 228.225502 64.112502) (end 228.569502 64.456502) (width 0.6) (layer "F.Cu") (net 9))
 (segment (start 247.963302 47.963302) (end 247.963302 50.483302) (width 0.6) (layer "F.Cu") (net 12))
 (segment (start 219.39 46) (end 246 46) (width 0.6) (layer "F.Cu") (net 12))
 (segment (start 250 56) (end 250 66.091004) (width 0.6) (layer "F.Cu") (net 12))
 (segment (start 247.963302 50.483302) (end 249.5 52.02) (width 0.6) (layer "F.Cu") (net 12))
 (segment (start 216.665502 40.525502) (end 216.665502 43.275502) (width 0.6) (layer "F.Cu") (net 12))
 (segment (start 245.465502 70.150102) (end 245.465502 70.625502) (width 0.6) (layer "F.Cu") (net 12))
 (segment (start 216.665502 43.275502) (end 219.39 46) (width 0.6) (layer "F.Cu") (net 12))
 (segment (start 250 66.091004) (end 245.465502 70.625502) (width 0.6) (layer "F.Cu") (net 12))
 (segment (start 246 46) (end 247.963302 47.963302) (width 0.6) (layer "F.Cu") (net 12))
 (segment (start 249.5 52.02) (end 249.5 55.5) (width 0.6) (layer "F.Cu") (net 12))
 (segment (start 249.5 55.5) (end 250 56) (width 0.6) (layer "F.Cu") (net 12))
 (segment (start 217.114502 47.974502) (end 233.604502 47.974502) (width 0.6) (layer "F.Cu") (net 10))
 (segment (start 212.165502 40.025502) (end 212.165502 43.025502) (width 0.6) (layer "F.Cu") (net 10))
 (segment (start 212.165502 43.025502) (end 217.114502 47.974502) (width 0.6) (layer "F.Cu") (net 10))
 (segment (start 233.604502 47.974502) (end 235.055502 49.425502) (width 0.6) (layer "F.Cu") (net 10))
 (segment (start 212.985502 62.805502) (end 212.985502 67.625502) (width 0.6) (layer "F.Cu") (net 15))
 (segment (start 214.911004 68.5) (end 214.911004 66.16) (width 0.6) (layer "F.Cu") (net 7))
 (segment (start 218.065502 63.005502) (end 220.417501 60.653503) (width 0.6) (layer "F.Cu") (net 7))
 (segment (start 229.867709 60.653503) (end 230.765502 61.551296) (width 0.6) (layer "F.Cu") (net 7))
 (segment (start 220.417501 60.653503) (end 229.867709 60.653503) (width 0.6) (layer "F.Cu") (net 7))
 (segment (start 230.765502 61.551296) (end 230.765502 63.005502) (width 0.6) (layer "F.Cu") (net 7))
 (segment (start 212.985502 70.425502) (end 214.911004 68.5) (width 0.6) (layer "F.Cu") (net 7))
 (segment (start 214.911004 66.16) (end 218.065502 63.005502) (width 0.6) (layer "F.Cu") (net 7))
 (segment (start 223 50.2) (end 217.508922 50.2) (width 0.6) (layer "F.Cu") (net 1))
 (segment (start 217.508922 50.2) (end 212.98342 54.725502) (width 0.6) (layer "F.Cu") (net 1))
 (segment (start 218.065502 60.465502) (end 218.7785 59.752504) (width 0.6) (layer "F.Cu") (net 6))
 (segment (start 232.035502 61.54709) (end 232.035502 63.005502) (width 0.6) (layer "F.Cu") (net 6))
 (segment (start 218.7785 59.752504) (end 230.240916 59.752504) (width 0.6) (layer "F.Cu") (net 6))
 (segment (start 230.240916 59.752504) (end 232.035502 61.54709) (width 0.6) (layer "F.Cu") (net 6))
 (segment (start 229.494502 61.554502) (end 225.945498 61.554502) (width 0.6) (layer "F.Cu") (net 8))
 (segment (start 221.954498 65.545502) (end 218.065502 65.545502) (width 0.6) (layer "F.Cu") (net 8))
 (segment (start 229.495502 61.555502) (end 229.494502 61.554502) (width 0.6) (layer "F.Cu") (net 8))
 (segment (start 225.945498 61.554502) (end 221.954498 65.545502) (width 0.6) (layer "F.Cu") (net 8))
 (segment (start 229.495502 63.005502) (end 229.495502 61.555502) (width 0.6) (layer "F.Cu") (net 8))
 (segment (start 229.495502 69.198502) (end 228.382502 68.085502) (width 0.6) (layer "F.Cu") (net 4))
 (segment (start 228.085502 68) (end 228 68.085502) (width 0.6) (layer "F.Cu") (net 4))
 (segment (start 230.846798 67.5) (end 229.495502 68.851296) (width 0.6) (layer "F.Cu") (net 4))
 (segment (start 241.5 67.5) (end 230.846798 67.5) (width 0.6) (layer "F.Cu") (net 4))
 (segment (start 228 68.085502) (end 218.065502 68.085502) (width 0.6) (layer "F.Cu") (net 4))
 (segment (start 246.005502 64.005502) (end 244.994498 64.005502) (width 0.6) (layer "F.Cu") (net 4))
 (segment (start 244.994498 64.005502) (end 241.5 67.5) (width 0.6) (layer "F.Cu") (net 4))
 (segment (start 229.495502 68.851296) (end 229.495502 69.198502) (width 0.6) (layer "F.Cu") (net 4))
 (segment (start 229.495502 70.305502) (end 229.495502 69.198502) (width 0.6) (layer "F.Cu") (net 4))
 (segment (start 228.382502 68.085502) (end 228 68.085502) (width 0.6) (layer "F.Cu") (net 4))
 (segment (start 241.694502 68.854502) (end 243.465502 70.625502) (width 0.6) (layer "F.Cu") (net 5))
 (segment (start 216.614502 72.076502) (end 216.614502 76.306526) (width 0.6) (layer "F.Cu") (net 5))
 (segment (start 218.065502 70.625502) (end 216.614502 72.076502) (width 0.6) (layer "F.Cu") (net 5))
 (segment (start 230.765502 68.855502) (end 230.766502 68.854502) (width 0.6) (layer "F.Cu") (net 5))
 (segment (start 230.765502 70.305502) (end 230.765502 68.855502) (width 0.6) (layer "F.Cu") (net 5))
 (segment (start 230.766502 68.854502) (end 241.694502 68.854502) (width 0.6) (layer "F.Cu") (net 5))
 (segment (start 216.614502 76.306526) (end 218.906976 78.599) (width 0.6) (layer "F.Cu") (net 5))
 (segment (start 226.697798 78.599) (end 230.765502 74.531296) (width 0.6) (layer "F.Cu") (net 5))
 (segment (start 218.906976 78.599) (end 226.697798 78.599) (width 0.6) (layer "F.Cu") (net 5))
 (segment (start 230.765502 74.531296) (end 230.765502 70.305502) (width 0.6) (layer "F.Cu") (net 5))
 (segment (start 228.225502 70.305502) (end 228.225502 72.274498) (width 0.6) (layer "F.Cu") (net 3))
 (segment (start 227.334498 73.165502) (end 218.065502 73.165502) (width 0.6) (layer "F.Cu") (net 3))
 (segment (start 228.225502 72.274498) (end 227.334498 73.165502) (width 0.6) (layer "F.Cu") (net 3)))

